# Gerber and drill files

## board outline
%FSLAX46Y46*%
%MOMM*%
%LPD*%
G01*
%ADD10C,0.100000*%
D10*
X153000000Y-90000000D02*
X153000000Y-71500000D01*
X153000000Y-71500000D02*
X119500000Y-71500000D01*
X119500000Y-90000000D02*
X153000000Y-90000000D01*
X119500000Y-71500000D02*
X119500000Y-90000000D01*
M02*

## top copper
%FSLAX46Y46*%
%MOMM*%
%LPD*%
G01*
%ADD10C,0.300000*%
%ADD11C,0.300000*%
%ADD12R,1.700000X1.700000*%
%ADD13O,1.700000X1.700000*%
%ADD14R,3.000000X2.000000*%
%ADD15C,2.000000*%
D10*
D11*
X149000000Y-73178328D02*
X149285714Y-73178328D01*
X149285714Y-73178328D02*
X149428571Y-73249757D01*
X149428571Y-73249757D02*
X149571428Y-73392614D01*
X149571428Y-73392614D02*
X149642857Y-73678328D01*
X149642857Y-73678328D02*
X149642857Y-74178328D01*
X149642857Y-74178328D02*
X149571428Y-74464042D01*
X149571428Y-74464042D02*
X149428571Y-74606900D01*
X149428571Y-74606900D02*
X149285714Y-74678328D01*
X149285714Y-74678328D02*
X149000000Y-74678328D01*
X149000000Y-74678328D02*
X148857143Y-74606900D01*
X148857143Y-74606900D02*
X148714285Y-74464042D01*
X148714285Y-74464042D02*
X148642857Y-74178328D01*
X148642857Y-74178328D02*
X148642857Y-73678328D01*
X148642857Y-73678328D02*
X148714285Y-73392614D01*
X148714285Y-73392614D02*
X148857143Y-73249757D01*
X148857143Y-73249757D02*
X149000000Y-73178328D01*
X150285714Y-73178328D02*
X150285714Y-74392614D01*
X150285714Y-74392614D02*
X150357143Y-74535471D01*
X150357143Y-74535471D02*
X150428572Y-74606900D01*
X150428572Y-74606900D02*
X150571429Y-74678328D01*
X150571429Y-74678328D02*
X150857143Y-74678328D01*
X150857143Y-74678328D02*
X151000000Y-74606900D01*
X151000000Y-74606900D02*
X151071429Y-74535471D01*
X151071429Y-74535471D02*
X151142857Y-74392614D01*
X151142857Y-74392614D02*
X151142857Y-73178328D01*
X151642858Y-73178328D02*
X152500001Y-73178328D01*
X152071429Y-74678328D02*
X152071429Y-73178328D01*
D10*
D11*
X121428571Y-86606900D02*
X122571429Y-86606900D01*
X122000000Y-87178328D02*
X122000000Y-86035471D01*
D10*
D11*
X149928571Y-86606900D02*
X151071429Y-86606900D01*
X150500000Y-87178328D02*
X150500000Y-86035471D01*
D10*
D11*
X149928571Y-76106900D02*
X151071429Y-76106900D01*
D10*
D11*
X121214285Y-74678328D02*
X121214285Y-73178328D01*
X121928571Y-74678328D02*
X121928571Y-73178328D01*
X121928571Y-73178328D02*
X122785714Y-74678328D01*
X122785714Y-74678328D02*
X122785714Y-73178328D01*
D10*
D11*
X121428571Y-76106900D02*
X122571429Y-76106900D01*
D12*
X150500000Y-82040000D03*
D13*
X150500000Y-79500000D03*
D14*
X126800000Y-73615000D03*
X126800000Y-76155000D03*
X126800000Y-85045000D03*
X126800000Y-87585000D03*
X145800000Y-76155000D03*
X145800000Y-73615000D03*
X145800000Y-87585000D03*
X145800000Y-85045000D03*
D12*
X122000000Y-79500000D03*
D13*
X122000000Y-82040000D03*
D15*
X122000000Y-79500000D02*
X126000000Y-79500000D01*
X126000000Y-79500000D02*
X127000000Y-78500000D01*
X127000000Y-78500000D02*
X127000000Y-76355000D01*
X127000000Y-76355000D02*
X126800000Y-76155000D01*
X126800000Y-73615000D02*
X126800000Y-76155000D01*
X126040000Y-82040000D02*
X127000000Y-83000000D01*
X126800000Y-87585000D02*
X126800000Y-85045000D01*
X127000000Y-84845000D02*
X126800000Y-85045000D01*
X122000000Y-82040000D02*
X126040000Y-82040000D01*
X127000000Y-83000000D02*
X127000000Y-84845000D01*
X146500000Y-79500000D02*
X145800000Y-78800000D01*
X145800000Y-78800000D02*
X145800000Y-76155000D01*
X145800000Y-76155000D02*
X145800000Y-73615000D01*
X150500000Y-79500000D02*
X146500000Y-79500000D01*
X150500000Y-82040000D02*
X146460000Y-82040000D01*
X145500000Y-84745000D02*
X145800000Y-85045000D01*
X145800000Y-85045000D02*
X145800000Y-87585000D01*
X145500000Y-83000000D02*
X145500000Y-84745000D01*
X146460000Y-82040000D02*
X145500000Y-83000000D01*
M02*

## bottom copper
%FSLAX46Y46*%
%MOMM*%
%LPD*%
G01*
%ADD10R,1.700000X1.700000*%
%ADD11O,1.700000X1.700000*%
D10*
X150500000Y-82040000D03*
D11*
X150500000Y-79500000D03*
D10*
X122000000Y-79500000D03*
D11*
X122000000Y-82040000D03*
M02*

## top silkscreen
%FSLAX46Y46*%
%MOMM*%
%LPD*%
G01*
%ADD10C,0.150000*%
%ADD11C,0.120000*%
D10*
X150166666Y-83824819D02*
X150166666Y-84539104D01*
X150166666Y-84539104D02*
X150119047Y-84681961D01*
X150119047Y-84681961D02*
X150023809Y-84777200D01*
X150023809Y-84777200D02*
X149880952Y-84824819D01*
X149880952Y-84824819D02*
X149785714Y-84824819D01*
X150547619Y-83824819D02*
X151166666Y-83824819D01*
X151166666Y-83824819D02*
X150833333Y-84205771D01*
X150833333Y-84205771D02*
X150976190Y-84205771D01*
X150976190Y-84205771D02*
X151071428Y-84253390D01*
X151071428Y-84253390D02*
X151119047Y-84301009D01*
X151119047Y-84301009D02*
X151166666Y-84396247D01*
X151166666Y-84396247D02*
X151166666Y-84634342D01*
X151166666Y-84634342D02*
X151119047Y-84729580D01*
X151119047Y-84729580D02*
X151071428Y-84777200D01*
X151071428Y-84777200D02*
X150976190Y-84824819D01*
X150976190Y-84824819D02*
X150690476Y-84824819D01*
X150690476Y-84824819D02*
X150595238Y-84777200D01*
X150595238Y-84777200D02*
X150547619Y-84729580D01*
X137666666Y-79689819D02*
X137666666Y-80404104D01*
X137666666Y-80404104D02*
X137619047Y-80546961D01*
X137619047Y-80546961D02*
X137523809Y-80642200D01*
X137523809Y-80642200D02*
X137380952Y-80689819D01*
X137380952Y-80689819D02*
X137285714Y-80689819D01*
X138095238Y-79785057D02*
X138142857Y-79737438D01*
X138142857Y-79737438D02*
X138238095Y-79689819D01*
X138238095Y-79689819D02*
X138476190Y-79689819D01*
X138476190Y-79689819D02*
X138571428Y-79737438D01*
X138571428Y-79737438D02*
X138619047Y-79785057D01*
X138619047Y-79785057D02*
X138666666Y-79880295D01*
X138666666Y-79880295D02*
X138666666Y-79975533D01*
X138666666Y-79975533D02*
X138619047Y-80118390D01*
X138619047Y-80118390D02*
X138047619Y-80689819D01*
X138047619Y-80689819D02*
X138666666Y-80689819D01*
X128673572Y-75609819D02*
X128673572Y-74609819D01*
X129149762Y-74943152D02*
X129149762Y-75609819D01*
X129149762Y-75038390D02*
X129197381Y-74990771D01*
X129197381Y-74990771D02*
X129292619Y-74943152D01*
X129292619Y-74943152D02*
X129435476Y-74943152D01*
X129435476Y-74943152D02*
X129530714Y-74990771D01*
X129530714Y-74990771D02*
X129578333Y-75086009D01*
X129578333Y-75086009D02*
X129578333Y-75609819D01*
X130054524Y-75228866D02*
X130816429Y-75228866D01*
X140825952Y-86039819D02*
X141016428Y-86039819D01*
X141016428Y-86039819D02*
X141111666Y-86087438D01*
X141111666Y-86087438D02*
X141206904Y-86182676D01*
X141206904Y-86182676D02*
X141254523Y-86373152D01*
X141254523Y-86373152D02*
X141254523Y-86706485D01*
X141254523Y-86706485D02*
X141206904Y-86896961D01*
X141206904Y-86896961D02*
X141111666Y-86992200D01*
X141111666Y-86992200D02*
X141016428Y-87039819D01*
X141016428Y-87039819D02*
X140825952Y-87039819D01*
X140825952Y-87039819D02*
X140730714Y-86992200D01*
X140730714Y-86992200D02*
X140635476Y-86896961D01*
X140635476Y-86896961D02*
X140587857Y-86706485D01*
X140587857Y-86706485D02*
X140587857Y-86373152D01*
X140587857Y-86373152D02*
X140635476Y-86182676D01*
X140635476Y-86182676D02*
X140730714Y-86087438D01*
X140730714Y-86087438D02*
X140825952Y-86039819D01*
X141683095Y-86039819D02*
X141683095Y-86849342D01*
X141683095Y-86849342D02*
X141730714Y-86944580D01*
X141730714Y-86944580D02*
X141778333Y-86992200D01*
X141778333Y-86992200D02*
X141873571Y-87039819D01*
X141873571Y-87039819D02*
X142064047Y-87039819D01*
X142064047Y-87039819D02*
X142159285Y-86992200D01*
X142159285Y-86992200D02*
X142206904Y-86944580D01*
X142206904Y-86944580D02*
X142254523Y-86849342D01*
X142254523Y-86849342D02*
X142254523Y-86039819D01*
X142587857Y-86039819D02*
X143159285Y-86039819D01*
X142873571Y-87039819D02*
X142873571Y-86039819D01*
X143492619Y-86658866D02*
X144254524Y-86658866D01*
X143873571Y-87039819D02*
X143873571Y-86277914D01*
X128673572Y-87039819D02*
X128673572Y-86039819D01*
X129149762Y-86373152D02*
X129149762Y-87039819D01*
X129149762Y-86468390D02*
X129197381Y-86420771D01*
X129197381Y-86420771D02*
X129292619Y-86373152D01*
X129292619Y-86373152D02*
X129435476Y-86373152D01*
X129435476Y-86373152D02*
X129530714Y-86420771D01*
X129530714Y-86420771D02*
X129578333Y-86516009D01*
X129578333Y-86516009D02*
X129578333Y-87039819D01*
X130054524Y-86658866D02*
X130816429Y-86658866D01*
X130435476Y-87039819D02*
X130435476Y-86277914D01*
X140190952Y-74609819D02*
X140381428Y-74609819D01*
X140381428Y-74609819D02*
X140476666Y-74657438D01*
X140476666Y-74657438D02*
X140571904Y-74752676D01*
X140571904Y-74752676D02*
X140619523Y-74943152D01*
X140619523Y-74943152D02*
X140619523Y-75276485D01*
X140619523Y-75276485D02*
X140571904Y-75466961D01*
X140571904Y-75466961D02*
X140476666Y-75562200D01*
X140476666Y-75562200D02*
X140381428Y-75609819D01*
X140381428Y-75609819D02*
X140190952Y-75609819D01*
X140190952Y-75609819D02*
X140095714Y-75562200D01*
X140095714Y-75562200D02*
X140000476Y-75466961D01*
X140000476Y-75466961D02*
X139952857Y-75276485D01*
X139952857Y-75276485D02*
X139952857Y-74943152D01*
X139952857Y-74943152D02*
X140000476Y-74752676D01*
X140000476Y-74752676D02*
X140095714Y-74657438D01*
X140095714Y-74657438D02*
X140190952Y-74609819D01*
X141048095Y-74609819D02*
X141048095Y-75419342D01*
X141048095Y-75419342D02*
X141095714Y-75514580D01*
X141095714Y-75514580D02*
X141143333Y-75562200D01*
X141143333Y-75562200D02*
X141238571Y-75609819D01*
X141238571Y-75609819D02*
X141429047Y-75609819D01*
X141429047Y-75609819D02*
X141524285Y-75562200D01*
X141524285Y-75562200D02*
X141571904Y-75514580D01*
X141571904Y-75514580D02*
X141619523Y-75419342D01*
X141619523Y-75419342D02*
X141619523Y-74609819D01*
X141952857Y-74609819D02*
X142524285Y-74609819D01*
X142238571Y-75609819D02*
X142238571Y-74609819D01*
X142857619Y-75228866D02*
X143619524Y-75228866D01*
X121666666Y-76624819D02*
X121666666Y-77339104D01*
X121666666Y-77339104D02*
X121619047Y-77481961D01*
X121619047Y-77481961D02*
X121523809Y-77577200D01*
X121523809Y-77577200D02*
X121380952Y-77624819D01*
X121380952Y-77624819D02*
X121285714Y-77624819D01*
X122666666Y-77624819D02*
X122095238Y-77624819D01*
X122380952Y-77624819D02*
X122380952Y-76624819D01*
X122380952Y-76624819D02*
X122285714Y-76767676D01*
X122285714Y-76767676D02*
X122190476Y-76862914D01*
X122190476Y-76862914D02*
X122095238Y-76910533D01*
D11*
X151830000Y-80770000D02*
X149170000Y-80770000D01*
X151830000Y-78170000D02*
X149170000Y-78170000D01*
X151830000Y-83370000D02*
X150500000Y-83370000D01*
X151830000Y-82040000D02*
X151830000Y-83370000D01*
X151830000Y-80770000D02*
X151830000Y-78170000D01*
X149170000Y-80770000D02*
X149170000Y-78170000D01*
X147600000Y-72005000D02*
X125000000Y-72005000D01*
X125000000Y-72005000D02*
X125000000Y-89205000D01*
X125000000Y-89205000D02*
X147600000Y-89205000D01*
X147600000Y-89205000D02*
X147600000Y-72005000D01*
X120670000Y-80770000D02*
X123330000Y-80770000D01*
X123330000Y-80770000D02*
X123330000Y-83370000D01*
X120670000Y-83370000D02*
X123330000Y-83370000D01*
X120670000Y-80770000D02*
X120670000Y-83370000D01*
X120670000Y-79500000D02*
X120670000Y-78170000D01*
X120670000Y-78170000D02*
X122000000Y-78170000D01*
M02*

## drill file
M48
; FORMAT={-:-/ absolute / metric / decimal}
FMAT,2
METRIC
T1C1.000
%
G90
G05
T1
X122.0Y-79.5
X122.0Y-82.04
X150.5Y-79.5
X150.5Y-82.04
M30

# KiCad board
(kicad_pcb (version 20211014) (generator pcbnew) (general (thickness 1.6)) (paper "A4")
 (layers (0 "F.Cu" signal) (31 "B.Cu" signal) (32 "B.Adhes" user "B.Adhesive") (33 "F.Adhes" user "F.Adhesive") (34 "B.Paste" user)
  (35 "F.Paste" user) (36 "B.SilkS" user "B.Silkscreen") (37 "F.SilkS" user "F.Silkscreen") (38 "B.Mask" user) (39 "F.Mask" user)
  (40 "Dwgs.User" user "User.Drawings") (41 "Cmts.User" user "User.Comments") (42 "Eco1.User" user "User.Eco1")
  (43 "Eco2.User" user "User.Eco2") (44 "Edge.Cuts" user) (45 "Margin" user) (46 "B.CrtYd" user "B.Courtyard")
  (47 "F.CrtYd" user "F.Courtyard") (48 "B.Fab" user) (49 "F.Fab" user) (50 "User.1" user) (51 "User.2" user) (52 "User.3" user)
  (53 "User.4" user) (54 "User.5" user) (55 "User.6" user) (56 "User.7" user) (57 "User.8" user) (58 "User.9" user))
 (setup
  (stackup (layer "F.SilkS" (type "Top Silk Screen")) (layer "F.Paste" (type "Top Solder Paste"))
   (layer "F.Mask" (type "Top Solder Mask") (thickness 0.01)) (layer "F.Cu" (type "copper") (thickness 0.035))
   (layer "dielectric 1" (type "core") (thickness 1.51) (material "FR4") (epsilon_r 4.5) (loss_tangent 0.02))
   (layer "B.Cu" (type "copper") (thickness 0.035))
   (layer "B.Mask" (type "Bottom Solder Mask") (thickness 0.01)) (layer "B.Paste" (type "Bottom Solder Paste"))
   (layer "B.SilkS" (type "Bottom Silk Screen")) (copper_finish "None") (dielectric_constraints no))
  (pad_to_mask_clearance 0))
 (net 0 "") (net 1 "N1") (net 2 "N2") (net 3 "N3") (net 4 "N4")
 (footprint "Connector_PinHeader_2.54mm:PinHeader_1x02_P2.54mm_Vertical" (layer "F.Cu") (at 150.5 82.04 180)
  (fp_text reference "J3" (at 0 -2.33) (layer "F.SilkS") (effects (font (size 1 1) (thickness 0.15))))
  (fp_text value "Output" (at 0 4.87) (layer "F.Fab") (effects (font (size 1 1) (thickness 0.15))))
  (fp_line (start -1.33 1.27) (end 1.33 1.27) (layer "F.SilkS") (width 0.12))
  (fp_line (start -1.33 3.87) (end 1.33 3.87) (layer "F.SilkS") (width 0.12))
  (fp_line (start -1.33 -1.33) (end 0 -1.33) (layer "F.SilkS") (width 0.12))
  (fp_line (start -1.33 0) (end -1.33 -1.33) (layer "F.SilkS") (width 0.12))
  (fp_line (start -1.33 1.27) (end -1.33 3.87) (layer "F.SilkS") (width 0.12))
  (fp_line (start 1.33 1.27) (end 1.33 3.87) (layer "F.SilkS") (width 0.12))
  (pad "1" thru_hole rect (at 0 0 180) (size 1.7 1.7) (drill 1) (layers *.Cu *.Mask) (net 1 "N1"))
  (pad "2" thru_hole oval (at 0 2.54 180) (size 1.7 1.7) (drill 1) (layers *.Cu *.Mask) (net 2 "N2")))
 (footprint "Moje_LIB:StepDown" (layer "F.Cu") (at 125 72)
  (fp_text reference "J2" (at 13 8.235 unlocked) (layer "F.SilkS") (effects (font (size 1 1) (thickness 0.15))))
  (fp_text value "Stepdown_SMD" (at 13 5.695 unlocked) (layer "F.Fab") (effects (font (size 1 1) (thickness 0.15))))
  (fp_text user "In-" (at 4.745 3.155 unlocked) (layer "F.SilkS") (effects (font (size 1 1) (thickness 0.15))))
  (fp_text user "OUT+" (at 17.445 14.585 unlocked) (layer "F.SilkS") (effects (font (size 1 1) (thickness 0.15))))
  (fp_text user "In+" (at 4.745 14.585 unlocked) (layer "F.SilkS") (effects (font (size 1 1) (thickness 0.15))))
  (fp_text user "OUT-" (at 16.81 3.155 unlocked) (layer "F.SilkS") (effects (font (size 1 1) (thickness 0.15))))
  (fp_line (start 22.6 0.005) (end 0 0.005) (layer "F.SilkS") (width 0.12))
  (fp_line (start 0 0.005) (end 0 17.205) (layer "F.SilkS") (width 0.12))
  (fp_line (start 0 17.205) (end 22.6 17.205) (layer "F.SilkS") (width 0.12))
  (fp_line (start 22.6 17.205) (end 22.6 0.005) (layer "F.SilkS") (width 0.12))
  (pad "1" smd rect (at 1.8 1.615) (size 3 2) (layers "F.Cu" "F.Paste" "F.Mask") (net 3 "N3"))
  (pad "1" smd rect (at 1.8 4.155) (size 3 2) (layers "F.Cu" "F.Paste" "F.Mask") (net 3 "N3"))
  (pad "2" smd rect (at 1.8 13.045) (size 3 2) (layers "F.Cu" "F.Paste" "F.Mask") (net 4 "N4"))
  (pad "2" smd rect (at 1.8 15.585) (size 3 2) (layers "F.Cu" "F.Paste" "F.Mask") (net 4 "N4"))
  (pad "3" smd rect (at 20.8 4.155) (size 3 2) (layers "F.Cu" "F.Paste" "F.Mask") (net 2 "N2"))
  (pad "3" smd rect (at 20.8 1.615) (size 3 2) (layers "F.Cu" "F.Paste" "F.Mask") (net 2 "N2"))
  (pad "4" smd rect (at 20.8 15.585) (size 3 2) (layers "F.Cu" "F.Paste" "F.Mask") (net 1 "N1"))
  (pad "4" smd rect (at 20.8 13.045) (size 3 2) (layers "F.Cu" "F.Paste" "F.Mask") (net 1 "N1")))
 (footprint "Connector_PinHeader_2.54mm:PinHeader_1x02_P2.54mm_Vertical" (layer "F.Cu") (at 122 79.5)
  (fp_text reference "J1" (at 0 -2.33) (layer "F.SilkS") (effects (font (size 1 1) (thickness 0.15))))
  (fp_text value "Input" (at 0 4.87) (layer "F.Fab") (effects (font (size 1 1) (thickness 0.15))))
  (fp_line (start -1.33 1.27) (end 1.33 1.27) (layer "F.SilkS") (width 0.12))
  (fp_line (start 1.33 1.27) (end 1.33 3.87) (layer "F.SilkS") (width 0.12))
  (fp_line (start -1.33 3.87) (end 1.33 3.87) (layer "F.SilkS") (width 0.12))
  (fp_line (start -1.33 1.27) (end -1.33 3.87) (layer "F.SilkS") (width 0.12))
  (fp_line (start -1.33 0) (end -1.33 -1.33) (layer "F.SilkS") (width 0.12))
  (fp_line (start -1.33 -1.33) (end 0 -1.33) (layer "F.SilkS") (width 0.12))
  (pad "1" thru_hole rect (at 0 0) (size 1.7 1.7) (drill 1) (layers *.Cu *.Mask) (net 3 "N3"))
  (pad "2" thru_hole oval (at 0 2.54) (size 1.7 1.7) (drill 1) (layers *.Cu *.Mask) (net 4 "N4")))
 (gr_line (start 153 90) (end 153 71.5) (layer "Edge.Cuts") (width 0.1))
 (gr_line (start 153 71.5) (end 119.5 71.5) (layer "Edge.Cuts") (width 0.1))
 (gr_line (start 119.5 90) (end 153 90) (layer "Edge.Cuts") (width 0.1))
 (gr_line (start 119.5 71.5) (end 119.5 90) (layer "Edge.Cuts") (width 0.1))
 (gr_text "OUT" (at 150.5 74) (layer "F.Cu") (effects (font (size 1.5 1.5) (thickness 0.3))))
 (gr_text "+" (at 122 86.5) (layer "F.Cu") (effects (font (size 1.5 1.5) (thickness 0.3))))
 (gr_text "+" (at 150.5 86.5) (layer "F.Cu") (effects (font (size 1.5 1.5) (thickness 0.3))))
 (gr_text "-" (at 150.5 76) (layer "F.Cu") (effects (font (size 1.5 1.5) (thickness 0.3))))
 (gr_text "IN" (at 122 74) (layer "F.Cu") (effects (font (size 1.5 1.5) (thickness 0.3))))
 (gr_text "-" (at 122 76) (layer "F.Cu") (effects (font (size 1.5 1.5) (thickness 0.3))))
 (segment (start 122 79.5) (end 126 79.5) (width 2) (layer "F.Cu") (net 3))
 (segment (start 126 79.5) (end 127 78.5) (width 2) (layer "F.Cu") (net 3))
 (segment (start 127 78.5) (end 127 76.355) (width 2) (layer "F.Cu") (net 3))
 (segment (start 127 76.355) (end 126.8 76.155) (width 2) (layer "F.Cu") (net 3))
 (segment (start 126.8 73.615) (end 126.8 76.155) (width 2) (layer "F.Cu") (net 3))
 (segment (start 126.04 82.04) (end 127 83) (width 2) (layer "F.Cu") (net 4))
 (segment (start 126.8 87.585) (end 126.8 85.045) (width 2) (layer "F.Cu") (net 4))
 (segment (start 127 84.845) (end 126.8 85.045) (width 2) (layer "F.Cu") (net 4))
 (segment (start 122 82.04) (end 126.04 82.04) (width 2) (layer "F.Cu") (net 4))
 (segment (start 127 83) (end 127 84.845) (width 2) (layer "F.Cu") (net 4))
 (segment (start 146.5 79.5) (end 145.8 78.8) (width 2) (layer "F.Cu") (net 2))
 (segment (start 145.8 78.8) (end 145.8 76.155) (width 2) (layer "F.Cu") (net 2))
 (segment (start 145.8 76.155) (end 145.8 73.615) (width 2) (layer "F.Cu") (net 2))
 (segment (start 150.5 79.5) (end 146.5 79.5) (width 2) (layer "F.Cu") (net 2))
 (segment (start 150.5 82.04) (end 146.46 82.04) (width 2) (layer "F.Cu") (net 1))
 (segment (start 145.5 84.745) (end 145.8 85.045) (width 2) (layer "F.Cu") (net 1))
 (segment (start 145.8 85.045) (end 145.8 87.585) (width 2) (layer "F.Cu") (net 1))
 (segment (start 145.5 83) (end 145.5 84.745) (width 2) (layer "F.Cu") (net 1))
 (segment (start 146.46 82.04) (end 145.5 83) (width 2) (layer "F.Cu") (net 1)))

